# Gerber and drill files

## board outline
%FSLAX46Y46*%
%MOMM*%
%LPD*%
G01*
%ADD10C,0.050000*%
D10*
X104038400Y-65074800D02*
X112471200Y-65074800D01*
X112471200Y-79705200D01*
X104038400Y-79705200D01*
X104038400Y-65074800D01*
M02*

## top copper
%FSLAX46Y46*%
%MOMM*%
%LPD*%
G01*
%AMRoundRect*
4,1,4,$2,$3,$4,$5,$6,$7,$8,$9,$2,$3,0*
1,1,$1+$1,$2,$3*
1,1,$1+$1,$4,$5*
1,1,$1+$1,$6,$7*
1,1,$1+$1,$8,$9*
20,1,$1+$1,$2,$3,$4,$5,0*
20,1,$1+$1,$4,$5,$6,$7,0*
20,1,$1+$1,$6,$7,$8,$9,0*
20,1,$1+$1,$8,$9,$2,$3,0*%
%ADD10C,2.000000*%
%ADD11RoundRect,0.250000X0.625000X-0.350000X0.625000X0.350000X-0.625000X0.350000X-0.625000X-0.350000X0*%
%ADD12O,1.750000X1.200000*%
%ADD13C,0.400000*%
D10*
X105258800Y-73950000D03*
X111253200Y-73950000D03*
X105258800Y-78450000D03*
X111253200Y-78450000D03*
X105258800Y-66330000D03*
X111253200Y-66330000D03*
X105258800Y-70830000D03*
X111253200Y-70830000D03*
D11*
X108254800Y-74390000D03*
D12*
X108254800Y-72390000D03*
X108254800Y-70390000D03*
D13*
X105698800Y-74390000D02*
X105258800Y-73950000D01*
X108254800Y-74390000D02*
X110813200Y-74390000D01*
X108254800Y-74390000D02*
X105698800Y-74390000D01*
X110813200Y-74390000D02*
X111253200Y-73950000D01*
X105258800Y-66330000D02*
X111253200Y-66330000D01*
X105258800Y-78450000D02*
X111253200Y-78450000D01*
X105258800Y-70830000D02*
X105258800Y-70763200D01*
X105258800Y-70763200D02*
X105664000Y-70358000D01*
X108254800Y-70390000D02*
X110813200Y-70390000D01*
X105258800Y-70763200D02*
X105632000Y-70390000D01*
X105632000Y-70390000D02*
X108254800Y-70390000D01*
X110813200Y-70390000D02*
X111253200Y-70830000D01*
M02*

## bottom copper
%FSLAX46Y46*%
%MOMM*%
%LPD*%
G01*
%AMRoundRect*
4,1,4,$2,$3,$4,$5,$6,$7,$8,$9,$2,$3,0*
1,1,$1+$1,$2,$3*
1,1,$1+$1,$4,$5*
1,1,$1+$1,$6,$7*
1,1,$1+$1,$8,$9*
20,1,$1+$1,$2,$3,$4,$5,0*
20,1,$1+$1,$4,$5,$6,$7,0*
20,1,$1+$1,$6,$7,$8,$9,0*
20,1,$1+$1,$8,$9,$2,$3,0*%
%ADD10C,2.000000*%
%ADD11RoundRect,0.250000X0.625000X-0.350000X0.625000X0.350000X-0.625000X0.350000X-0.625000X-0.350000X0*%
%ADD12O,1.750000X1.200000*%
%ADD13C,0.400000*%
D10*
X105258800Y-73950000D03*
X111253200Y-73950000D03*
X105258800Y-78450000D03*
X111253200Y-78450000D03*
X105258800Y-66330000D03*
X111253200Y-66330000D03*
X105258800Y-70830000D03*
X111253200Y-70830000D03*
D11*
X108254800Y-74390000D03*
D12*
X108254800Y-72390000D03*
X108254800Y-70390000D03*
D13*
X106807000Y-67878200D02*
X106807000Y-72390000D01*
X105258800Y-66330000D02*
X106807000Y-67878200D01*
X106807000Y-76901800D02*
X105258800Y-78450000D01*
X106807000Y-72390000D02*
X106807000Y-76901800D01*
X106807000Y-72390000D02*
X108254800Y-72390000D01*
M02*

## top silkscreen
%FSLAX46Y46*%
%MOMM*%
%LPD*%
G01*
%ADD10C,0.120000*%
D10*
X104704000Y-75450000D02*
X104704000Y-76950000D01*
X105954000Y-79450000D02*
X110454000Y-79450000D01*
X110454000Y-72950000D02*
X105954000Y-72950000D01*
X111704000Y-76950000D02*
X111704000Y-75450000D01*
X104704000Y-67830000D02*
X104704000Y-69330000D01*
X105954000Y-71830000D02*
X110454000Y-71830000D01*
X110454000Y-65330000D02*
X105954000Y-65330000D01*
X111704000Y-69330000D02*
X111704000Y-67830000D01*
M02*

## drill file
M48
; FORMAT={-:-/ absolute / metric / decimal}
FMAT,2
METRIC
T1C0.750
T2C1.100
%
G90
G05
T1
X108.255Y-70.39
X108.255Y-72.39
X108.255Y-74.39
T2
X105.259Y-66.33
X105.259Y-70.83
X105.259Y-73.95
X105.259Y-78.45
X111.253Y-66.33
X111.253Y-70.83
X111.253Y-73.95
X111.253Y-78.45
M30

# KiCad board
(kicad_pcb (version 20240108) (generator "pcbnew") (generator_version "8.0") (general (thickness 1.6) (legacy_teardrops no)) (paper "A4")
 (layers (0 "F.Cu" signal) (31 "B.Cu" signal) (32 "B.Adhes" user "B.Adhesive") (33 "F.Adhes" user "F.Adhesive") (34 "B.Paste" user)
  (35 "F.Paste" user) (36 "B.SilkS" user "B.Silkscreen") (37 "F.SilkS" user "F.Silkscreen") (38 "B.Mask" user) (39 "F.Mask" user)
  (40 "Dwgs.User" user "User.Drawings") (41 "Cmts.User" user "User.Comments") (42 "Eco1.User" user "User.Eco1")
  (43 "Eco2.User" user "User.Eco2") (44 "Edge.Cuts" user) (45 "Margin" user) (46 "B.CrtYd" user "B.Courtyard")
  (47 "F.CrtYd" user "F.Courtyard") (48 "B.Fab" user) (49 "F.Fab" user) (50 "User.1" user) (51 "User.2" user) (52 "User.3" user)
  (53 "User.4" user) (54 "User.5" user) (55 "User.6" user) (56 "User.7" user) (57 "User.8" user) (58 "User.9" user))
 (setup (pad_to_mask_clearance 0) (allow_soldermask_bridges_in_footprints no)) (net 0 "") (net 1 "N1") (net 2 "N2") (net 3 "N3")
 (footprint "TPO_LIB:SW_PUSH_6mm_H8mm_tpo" (layer "F.Cu") (at 108.204 76.2)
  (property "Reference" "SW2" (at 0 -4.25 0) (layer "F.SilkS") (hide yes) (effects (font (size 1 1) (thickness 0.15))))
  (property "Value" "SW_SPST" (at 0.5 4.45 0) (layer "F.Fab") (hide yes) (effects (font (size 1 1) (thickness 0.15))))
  (fp_line (start -3.5 -0.75) (end -3.5 0.75) (stroke (width 0.12) (type solid)) (layer "F.SilkS"))
  (fp_line (start -2.25 3.25) (end 2.25 3.25) (stroke (width 0.12) (type solid)) (layer "F.SilkS"))
  (fp_line (start 2.25 -3.25) (end -2.25 -3.25) (stroke (width 0.12) (type solid)) (layer "F.SilkS"))
  (fp_line (start 3.5 0.75) (end 3.5 -0.75) (stroke (width 0.12) (type solid)) (layer "F.SilkS"))
  (pad "1" thru_hole circle (at -2.9452 -2.25 90) (size 2 2) (drill 1.1) (layers "*.Cu" "*.Mask") (remove_unused_layers no) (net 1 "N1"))
  (pad "1" thru_hole circle (at 3.0492 -2.25 90) (size 2 2) (drill 1.1) (layers "*.Cu" "*.Mask") (remove_unused_layers no) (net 1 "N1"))
  (pad "2" thru_hole circle (at -2.9452 2.25 90) (size 2 2) (drill 1.1) (layers "*.Cu" "*.Mask") (remove_unused_layers no) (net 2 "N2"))
  (pad "2" thru_hole circle (at 3.0492 2.25 90) (size 2 2) (drill 1.1) (layers "*.Cu" "*.Mask") (remove_unused_layers no) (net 2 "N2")))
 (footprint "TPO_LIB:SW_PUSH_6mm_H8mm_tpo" (layer "F.Cu") (at 108.204 68.58)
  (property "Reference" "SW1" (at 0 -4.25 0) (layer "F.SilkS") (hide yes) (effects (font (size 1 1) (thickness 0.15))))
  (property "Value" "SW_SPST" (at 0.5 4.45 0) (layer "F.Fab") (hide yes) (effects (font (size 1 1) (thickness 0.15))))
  (fp_line (start -3.5 -0.75) (end -3.5 0.75) (stroke (width 0.12) (type solid)) (layer "F.SilkS"))
  (fp_line (start -2.25 3.25) (end 2.25 3.25) (stroke (width 0.12) (type solid)) (layer "F.SilkS"))
  (fp_line (start 2.25 -3.25) (end -2.25 -3.25) (stroke (width 0.12) (type solid)) (layer "F.SilkS"))
  (fp_line (start 3.5 0.75) (end 3.5 -0.75) (stroke (width 0.12) (type solid)) (layer "F.SilkS"))
  (pad "1" thru_hole circle (at -2.9452 -2.25 90) (size 2 2) (drill 1.1) (layers "*.Cu" "*.Mask") (remove_unused_layers no) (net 2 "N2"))
  (pad "1" thru_hole circle (at 3.0492 -2.25 90) (size 2 2) (drill 1.1) (layers "*.Cu" "*.Mask") (remove_unused_layers no) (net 2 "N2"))
  (pad "2" thru_hole circle (at -2.9452 2.25 90) (size 2 2) (drill 1.1) (layers "*.Cu" "*.Mask") (remove_unused_layers no) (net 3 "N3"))
  (pad "2" thru_hole circle (at 3.0492 2.25 90) (size 2 2) (drill 1.1) (layers "*.Cu" "*.Mask") (remove_unused_layers no) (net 3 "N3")))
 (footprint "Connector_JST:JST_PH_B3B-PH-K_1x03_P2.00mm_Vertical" (layer "B.Cu") (at 108.2548 74.39 90)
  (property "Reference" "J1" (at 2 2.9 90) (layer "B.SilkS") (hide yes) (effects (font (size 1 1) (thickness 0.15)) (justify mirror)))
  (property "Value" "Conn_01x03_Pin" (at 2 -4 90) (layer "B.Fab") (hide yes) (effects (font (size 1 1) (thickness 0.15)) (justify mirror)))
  (pad "1" thru_hole roundrect (at 0 0 90) (size 1.2 1.75) (drill 0.75) (layers "*.Cu" "*.Mask") (remove_unused_layers no)
   (roundrect_rratio 0.208333) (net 1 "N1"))
  (pad "2" thru_hole oval (at 2 0 90) (size 1.2 1.75) (drill 0.75) (layers "*.Cu" "*.Mask") (remove_unused_layers no) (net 2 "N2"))
  (pad "3" thru_hole oval (at 4 0 90) (size 1.2 1.75) (drill 0.75) (layers "*.Cu" "*.Mask") (remove_unused_layers no) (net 3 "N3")))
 (gr_rect (start 104.0384 65.0748) (end 112.4712 79.7052) (stroke (width 0.05) (type default)) (fill none) (layer "Edge.Cuts"))
 (segment (start 105.6988 74.39) (end 105.2588 73.95) (width 0.4) (layer "F.Cu") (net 1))
 (segment (start 108.2548 74.39) (end 110.8132 74.39) (width 0.4) (layer "F.Cu") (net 1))
 (segment (start 108.2548 74.39) (end 105.6988 74.39) (width 0.4) (layer "F.Cu") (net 1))
 (segment (start 110.8132 74.39) (end 111.2532 73.95) (width 0.4) (layer "F.Cu") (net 1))
 (segment (start 105.2588 66.33) (end 111.2532 66.33) (width 0.4) (layer "F.Cu") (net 2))
 (segment (start 105.2588 78.45) (end 111.2532 78.45) (width 0.4) (layer "F.Cu") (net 2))
 (segment (start 106.807 67.8782) (end 106.807 72.39) (width 0.4) (layer "B.Cu") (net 2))
 (segment (start 105.2588 66.33) (end 106.807 67.8782) (width 0.4) (layer "B.Cu") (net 2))
 (segment (start 106.807 76.9018) (end 105.2588 78.45) (width 0.4) (layer "B.Cu") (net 2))
 (segment (start 106.807 72.39) (end 106.807 76.9018) (width 0.4) (layer "B.Cu") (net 2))
 (segment (start 106.807 72.39) (end 108.2548 72.39) (width 0.4) (layer "B.Cu") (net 2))
 (segment (start 105.2588 70.83) (end 105.2588 70.7632) (width 0.4) (layer "F.Cu") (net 3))
 (segment (start 105.2588 70.7632) (end 105.664 70.358) (width 0.4) (layer "F.Cu") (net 3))
 (segment (start 108.2548 70.39) (end 110.8132 70.39) (width 0.4) (layer "F.Cu") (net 3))
 (segment (start 105.2588 70.7632) (end 105.632 70.39) (width 0.4) (layer "F.Cu") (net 3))
 (segment (start 105.632 70.39) (end 108.2548 70.39) (width 0.4) (layer "F.Cu") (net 3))
 (segment (start 110.8132 70.39) (end 111.2532 70.83) (width 0.4) (layer "F.Cu") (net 3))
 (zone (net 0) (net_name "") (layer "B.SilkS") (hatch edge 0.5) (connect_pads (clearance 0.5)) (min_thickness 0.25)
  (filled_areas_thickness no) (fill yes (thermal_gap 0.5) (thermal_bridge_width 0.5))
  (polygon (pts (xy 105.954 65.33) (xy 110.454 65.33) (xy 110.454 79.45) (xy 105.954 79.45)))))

